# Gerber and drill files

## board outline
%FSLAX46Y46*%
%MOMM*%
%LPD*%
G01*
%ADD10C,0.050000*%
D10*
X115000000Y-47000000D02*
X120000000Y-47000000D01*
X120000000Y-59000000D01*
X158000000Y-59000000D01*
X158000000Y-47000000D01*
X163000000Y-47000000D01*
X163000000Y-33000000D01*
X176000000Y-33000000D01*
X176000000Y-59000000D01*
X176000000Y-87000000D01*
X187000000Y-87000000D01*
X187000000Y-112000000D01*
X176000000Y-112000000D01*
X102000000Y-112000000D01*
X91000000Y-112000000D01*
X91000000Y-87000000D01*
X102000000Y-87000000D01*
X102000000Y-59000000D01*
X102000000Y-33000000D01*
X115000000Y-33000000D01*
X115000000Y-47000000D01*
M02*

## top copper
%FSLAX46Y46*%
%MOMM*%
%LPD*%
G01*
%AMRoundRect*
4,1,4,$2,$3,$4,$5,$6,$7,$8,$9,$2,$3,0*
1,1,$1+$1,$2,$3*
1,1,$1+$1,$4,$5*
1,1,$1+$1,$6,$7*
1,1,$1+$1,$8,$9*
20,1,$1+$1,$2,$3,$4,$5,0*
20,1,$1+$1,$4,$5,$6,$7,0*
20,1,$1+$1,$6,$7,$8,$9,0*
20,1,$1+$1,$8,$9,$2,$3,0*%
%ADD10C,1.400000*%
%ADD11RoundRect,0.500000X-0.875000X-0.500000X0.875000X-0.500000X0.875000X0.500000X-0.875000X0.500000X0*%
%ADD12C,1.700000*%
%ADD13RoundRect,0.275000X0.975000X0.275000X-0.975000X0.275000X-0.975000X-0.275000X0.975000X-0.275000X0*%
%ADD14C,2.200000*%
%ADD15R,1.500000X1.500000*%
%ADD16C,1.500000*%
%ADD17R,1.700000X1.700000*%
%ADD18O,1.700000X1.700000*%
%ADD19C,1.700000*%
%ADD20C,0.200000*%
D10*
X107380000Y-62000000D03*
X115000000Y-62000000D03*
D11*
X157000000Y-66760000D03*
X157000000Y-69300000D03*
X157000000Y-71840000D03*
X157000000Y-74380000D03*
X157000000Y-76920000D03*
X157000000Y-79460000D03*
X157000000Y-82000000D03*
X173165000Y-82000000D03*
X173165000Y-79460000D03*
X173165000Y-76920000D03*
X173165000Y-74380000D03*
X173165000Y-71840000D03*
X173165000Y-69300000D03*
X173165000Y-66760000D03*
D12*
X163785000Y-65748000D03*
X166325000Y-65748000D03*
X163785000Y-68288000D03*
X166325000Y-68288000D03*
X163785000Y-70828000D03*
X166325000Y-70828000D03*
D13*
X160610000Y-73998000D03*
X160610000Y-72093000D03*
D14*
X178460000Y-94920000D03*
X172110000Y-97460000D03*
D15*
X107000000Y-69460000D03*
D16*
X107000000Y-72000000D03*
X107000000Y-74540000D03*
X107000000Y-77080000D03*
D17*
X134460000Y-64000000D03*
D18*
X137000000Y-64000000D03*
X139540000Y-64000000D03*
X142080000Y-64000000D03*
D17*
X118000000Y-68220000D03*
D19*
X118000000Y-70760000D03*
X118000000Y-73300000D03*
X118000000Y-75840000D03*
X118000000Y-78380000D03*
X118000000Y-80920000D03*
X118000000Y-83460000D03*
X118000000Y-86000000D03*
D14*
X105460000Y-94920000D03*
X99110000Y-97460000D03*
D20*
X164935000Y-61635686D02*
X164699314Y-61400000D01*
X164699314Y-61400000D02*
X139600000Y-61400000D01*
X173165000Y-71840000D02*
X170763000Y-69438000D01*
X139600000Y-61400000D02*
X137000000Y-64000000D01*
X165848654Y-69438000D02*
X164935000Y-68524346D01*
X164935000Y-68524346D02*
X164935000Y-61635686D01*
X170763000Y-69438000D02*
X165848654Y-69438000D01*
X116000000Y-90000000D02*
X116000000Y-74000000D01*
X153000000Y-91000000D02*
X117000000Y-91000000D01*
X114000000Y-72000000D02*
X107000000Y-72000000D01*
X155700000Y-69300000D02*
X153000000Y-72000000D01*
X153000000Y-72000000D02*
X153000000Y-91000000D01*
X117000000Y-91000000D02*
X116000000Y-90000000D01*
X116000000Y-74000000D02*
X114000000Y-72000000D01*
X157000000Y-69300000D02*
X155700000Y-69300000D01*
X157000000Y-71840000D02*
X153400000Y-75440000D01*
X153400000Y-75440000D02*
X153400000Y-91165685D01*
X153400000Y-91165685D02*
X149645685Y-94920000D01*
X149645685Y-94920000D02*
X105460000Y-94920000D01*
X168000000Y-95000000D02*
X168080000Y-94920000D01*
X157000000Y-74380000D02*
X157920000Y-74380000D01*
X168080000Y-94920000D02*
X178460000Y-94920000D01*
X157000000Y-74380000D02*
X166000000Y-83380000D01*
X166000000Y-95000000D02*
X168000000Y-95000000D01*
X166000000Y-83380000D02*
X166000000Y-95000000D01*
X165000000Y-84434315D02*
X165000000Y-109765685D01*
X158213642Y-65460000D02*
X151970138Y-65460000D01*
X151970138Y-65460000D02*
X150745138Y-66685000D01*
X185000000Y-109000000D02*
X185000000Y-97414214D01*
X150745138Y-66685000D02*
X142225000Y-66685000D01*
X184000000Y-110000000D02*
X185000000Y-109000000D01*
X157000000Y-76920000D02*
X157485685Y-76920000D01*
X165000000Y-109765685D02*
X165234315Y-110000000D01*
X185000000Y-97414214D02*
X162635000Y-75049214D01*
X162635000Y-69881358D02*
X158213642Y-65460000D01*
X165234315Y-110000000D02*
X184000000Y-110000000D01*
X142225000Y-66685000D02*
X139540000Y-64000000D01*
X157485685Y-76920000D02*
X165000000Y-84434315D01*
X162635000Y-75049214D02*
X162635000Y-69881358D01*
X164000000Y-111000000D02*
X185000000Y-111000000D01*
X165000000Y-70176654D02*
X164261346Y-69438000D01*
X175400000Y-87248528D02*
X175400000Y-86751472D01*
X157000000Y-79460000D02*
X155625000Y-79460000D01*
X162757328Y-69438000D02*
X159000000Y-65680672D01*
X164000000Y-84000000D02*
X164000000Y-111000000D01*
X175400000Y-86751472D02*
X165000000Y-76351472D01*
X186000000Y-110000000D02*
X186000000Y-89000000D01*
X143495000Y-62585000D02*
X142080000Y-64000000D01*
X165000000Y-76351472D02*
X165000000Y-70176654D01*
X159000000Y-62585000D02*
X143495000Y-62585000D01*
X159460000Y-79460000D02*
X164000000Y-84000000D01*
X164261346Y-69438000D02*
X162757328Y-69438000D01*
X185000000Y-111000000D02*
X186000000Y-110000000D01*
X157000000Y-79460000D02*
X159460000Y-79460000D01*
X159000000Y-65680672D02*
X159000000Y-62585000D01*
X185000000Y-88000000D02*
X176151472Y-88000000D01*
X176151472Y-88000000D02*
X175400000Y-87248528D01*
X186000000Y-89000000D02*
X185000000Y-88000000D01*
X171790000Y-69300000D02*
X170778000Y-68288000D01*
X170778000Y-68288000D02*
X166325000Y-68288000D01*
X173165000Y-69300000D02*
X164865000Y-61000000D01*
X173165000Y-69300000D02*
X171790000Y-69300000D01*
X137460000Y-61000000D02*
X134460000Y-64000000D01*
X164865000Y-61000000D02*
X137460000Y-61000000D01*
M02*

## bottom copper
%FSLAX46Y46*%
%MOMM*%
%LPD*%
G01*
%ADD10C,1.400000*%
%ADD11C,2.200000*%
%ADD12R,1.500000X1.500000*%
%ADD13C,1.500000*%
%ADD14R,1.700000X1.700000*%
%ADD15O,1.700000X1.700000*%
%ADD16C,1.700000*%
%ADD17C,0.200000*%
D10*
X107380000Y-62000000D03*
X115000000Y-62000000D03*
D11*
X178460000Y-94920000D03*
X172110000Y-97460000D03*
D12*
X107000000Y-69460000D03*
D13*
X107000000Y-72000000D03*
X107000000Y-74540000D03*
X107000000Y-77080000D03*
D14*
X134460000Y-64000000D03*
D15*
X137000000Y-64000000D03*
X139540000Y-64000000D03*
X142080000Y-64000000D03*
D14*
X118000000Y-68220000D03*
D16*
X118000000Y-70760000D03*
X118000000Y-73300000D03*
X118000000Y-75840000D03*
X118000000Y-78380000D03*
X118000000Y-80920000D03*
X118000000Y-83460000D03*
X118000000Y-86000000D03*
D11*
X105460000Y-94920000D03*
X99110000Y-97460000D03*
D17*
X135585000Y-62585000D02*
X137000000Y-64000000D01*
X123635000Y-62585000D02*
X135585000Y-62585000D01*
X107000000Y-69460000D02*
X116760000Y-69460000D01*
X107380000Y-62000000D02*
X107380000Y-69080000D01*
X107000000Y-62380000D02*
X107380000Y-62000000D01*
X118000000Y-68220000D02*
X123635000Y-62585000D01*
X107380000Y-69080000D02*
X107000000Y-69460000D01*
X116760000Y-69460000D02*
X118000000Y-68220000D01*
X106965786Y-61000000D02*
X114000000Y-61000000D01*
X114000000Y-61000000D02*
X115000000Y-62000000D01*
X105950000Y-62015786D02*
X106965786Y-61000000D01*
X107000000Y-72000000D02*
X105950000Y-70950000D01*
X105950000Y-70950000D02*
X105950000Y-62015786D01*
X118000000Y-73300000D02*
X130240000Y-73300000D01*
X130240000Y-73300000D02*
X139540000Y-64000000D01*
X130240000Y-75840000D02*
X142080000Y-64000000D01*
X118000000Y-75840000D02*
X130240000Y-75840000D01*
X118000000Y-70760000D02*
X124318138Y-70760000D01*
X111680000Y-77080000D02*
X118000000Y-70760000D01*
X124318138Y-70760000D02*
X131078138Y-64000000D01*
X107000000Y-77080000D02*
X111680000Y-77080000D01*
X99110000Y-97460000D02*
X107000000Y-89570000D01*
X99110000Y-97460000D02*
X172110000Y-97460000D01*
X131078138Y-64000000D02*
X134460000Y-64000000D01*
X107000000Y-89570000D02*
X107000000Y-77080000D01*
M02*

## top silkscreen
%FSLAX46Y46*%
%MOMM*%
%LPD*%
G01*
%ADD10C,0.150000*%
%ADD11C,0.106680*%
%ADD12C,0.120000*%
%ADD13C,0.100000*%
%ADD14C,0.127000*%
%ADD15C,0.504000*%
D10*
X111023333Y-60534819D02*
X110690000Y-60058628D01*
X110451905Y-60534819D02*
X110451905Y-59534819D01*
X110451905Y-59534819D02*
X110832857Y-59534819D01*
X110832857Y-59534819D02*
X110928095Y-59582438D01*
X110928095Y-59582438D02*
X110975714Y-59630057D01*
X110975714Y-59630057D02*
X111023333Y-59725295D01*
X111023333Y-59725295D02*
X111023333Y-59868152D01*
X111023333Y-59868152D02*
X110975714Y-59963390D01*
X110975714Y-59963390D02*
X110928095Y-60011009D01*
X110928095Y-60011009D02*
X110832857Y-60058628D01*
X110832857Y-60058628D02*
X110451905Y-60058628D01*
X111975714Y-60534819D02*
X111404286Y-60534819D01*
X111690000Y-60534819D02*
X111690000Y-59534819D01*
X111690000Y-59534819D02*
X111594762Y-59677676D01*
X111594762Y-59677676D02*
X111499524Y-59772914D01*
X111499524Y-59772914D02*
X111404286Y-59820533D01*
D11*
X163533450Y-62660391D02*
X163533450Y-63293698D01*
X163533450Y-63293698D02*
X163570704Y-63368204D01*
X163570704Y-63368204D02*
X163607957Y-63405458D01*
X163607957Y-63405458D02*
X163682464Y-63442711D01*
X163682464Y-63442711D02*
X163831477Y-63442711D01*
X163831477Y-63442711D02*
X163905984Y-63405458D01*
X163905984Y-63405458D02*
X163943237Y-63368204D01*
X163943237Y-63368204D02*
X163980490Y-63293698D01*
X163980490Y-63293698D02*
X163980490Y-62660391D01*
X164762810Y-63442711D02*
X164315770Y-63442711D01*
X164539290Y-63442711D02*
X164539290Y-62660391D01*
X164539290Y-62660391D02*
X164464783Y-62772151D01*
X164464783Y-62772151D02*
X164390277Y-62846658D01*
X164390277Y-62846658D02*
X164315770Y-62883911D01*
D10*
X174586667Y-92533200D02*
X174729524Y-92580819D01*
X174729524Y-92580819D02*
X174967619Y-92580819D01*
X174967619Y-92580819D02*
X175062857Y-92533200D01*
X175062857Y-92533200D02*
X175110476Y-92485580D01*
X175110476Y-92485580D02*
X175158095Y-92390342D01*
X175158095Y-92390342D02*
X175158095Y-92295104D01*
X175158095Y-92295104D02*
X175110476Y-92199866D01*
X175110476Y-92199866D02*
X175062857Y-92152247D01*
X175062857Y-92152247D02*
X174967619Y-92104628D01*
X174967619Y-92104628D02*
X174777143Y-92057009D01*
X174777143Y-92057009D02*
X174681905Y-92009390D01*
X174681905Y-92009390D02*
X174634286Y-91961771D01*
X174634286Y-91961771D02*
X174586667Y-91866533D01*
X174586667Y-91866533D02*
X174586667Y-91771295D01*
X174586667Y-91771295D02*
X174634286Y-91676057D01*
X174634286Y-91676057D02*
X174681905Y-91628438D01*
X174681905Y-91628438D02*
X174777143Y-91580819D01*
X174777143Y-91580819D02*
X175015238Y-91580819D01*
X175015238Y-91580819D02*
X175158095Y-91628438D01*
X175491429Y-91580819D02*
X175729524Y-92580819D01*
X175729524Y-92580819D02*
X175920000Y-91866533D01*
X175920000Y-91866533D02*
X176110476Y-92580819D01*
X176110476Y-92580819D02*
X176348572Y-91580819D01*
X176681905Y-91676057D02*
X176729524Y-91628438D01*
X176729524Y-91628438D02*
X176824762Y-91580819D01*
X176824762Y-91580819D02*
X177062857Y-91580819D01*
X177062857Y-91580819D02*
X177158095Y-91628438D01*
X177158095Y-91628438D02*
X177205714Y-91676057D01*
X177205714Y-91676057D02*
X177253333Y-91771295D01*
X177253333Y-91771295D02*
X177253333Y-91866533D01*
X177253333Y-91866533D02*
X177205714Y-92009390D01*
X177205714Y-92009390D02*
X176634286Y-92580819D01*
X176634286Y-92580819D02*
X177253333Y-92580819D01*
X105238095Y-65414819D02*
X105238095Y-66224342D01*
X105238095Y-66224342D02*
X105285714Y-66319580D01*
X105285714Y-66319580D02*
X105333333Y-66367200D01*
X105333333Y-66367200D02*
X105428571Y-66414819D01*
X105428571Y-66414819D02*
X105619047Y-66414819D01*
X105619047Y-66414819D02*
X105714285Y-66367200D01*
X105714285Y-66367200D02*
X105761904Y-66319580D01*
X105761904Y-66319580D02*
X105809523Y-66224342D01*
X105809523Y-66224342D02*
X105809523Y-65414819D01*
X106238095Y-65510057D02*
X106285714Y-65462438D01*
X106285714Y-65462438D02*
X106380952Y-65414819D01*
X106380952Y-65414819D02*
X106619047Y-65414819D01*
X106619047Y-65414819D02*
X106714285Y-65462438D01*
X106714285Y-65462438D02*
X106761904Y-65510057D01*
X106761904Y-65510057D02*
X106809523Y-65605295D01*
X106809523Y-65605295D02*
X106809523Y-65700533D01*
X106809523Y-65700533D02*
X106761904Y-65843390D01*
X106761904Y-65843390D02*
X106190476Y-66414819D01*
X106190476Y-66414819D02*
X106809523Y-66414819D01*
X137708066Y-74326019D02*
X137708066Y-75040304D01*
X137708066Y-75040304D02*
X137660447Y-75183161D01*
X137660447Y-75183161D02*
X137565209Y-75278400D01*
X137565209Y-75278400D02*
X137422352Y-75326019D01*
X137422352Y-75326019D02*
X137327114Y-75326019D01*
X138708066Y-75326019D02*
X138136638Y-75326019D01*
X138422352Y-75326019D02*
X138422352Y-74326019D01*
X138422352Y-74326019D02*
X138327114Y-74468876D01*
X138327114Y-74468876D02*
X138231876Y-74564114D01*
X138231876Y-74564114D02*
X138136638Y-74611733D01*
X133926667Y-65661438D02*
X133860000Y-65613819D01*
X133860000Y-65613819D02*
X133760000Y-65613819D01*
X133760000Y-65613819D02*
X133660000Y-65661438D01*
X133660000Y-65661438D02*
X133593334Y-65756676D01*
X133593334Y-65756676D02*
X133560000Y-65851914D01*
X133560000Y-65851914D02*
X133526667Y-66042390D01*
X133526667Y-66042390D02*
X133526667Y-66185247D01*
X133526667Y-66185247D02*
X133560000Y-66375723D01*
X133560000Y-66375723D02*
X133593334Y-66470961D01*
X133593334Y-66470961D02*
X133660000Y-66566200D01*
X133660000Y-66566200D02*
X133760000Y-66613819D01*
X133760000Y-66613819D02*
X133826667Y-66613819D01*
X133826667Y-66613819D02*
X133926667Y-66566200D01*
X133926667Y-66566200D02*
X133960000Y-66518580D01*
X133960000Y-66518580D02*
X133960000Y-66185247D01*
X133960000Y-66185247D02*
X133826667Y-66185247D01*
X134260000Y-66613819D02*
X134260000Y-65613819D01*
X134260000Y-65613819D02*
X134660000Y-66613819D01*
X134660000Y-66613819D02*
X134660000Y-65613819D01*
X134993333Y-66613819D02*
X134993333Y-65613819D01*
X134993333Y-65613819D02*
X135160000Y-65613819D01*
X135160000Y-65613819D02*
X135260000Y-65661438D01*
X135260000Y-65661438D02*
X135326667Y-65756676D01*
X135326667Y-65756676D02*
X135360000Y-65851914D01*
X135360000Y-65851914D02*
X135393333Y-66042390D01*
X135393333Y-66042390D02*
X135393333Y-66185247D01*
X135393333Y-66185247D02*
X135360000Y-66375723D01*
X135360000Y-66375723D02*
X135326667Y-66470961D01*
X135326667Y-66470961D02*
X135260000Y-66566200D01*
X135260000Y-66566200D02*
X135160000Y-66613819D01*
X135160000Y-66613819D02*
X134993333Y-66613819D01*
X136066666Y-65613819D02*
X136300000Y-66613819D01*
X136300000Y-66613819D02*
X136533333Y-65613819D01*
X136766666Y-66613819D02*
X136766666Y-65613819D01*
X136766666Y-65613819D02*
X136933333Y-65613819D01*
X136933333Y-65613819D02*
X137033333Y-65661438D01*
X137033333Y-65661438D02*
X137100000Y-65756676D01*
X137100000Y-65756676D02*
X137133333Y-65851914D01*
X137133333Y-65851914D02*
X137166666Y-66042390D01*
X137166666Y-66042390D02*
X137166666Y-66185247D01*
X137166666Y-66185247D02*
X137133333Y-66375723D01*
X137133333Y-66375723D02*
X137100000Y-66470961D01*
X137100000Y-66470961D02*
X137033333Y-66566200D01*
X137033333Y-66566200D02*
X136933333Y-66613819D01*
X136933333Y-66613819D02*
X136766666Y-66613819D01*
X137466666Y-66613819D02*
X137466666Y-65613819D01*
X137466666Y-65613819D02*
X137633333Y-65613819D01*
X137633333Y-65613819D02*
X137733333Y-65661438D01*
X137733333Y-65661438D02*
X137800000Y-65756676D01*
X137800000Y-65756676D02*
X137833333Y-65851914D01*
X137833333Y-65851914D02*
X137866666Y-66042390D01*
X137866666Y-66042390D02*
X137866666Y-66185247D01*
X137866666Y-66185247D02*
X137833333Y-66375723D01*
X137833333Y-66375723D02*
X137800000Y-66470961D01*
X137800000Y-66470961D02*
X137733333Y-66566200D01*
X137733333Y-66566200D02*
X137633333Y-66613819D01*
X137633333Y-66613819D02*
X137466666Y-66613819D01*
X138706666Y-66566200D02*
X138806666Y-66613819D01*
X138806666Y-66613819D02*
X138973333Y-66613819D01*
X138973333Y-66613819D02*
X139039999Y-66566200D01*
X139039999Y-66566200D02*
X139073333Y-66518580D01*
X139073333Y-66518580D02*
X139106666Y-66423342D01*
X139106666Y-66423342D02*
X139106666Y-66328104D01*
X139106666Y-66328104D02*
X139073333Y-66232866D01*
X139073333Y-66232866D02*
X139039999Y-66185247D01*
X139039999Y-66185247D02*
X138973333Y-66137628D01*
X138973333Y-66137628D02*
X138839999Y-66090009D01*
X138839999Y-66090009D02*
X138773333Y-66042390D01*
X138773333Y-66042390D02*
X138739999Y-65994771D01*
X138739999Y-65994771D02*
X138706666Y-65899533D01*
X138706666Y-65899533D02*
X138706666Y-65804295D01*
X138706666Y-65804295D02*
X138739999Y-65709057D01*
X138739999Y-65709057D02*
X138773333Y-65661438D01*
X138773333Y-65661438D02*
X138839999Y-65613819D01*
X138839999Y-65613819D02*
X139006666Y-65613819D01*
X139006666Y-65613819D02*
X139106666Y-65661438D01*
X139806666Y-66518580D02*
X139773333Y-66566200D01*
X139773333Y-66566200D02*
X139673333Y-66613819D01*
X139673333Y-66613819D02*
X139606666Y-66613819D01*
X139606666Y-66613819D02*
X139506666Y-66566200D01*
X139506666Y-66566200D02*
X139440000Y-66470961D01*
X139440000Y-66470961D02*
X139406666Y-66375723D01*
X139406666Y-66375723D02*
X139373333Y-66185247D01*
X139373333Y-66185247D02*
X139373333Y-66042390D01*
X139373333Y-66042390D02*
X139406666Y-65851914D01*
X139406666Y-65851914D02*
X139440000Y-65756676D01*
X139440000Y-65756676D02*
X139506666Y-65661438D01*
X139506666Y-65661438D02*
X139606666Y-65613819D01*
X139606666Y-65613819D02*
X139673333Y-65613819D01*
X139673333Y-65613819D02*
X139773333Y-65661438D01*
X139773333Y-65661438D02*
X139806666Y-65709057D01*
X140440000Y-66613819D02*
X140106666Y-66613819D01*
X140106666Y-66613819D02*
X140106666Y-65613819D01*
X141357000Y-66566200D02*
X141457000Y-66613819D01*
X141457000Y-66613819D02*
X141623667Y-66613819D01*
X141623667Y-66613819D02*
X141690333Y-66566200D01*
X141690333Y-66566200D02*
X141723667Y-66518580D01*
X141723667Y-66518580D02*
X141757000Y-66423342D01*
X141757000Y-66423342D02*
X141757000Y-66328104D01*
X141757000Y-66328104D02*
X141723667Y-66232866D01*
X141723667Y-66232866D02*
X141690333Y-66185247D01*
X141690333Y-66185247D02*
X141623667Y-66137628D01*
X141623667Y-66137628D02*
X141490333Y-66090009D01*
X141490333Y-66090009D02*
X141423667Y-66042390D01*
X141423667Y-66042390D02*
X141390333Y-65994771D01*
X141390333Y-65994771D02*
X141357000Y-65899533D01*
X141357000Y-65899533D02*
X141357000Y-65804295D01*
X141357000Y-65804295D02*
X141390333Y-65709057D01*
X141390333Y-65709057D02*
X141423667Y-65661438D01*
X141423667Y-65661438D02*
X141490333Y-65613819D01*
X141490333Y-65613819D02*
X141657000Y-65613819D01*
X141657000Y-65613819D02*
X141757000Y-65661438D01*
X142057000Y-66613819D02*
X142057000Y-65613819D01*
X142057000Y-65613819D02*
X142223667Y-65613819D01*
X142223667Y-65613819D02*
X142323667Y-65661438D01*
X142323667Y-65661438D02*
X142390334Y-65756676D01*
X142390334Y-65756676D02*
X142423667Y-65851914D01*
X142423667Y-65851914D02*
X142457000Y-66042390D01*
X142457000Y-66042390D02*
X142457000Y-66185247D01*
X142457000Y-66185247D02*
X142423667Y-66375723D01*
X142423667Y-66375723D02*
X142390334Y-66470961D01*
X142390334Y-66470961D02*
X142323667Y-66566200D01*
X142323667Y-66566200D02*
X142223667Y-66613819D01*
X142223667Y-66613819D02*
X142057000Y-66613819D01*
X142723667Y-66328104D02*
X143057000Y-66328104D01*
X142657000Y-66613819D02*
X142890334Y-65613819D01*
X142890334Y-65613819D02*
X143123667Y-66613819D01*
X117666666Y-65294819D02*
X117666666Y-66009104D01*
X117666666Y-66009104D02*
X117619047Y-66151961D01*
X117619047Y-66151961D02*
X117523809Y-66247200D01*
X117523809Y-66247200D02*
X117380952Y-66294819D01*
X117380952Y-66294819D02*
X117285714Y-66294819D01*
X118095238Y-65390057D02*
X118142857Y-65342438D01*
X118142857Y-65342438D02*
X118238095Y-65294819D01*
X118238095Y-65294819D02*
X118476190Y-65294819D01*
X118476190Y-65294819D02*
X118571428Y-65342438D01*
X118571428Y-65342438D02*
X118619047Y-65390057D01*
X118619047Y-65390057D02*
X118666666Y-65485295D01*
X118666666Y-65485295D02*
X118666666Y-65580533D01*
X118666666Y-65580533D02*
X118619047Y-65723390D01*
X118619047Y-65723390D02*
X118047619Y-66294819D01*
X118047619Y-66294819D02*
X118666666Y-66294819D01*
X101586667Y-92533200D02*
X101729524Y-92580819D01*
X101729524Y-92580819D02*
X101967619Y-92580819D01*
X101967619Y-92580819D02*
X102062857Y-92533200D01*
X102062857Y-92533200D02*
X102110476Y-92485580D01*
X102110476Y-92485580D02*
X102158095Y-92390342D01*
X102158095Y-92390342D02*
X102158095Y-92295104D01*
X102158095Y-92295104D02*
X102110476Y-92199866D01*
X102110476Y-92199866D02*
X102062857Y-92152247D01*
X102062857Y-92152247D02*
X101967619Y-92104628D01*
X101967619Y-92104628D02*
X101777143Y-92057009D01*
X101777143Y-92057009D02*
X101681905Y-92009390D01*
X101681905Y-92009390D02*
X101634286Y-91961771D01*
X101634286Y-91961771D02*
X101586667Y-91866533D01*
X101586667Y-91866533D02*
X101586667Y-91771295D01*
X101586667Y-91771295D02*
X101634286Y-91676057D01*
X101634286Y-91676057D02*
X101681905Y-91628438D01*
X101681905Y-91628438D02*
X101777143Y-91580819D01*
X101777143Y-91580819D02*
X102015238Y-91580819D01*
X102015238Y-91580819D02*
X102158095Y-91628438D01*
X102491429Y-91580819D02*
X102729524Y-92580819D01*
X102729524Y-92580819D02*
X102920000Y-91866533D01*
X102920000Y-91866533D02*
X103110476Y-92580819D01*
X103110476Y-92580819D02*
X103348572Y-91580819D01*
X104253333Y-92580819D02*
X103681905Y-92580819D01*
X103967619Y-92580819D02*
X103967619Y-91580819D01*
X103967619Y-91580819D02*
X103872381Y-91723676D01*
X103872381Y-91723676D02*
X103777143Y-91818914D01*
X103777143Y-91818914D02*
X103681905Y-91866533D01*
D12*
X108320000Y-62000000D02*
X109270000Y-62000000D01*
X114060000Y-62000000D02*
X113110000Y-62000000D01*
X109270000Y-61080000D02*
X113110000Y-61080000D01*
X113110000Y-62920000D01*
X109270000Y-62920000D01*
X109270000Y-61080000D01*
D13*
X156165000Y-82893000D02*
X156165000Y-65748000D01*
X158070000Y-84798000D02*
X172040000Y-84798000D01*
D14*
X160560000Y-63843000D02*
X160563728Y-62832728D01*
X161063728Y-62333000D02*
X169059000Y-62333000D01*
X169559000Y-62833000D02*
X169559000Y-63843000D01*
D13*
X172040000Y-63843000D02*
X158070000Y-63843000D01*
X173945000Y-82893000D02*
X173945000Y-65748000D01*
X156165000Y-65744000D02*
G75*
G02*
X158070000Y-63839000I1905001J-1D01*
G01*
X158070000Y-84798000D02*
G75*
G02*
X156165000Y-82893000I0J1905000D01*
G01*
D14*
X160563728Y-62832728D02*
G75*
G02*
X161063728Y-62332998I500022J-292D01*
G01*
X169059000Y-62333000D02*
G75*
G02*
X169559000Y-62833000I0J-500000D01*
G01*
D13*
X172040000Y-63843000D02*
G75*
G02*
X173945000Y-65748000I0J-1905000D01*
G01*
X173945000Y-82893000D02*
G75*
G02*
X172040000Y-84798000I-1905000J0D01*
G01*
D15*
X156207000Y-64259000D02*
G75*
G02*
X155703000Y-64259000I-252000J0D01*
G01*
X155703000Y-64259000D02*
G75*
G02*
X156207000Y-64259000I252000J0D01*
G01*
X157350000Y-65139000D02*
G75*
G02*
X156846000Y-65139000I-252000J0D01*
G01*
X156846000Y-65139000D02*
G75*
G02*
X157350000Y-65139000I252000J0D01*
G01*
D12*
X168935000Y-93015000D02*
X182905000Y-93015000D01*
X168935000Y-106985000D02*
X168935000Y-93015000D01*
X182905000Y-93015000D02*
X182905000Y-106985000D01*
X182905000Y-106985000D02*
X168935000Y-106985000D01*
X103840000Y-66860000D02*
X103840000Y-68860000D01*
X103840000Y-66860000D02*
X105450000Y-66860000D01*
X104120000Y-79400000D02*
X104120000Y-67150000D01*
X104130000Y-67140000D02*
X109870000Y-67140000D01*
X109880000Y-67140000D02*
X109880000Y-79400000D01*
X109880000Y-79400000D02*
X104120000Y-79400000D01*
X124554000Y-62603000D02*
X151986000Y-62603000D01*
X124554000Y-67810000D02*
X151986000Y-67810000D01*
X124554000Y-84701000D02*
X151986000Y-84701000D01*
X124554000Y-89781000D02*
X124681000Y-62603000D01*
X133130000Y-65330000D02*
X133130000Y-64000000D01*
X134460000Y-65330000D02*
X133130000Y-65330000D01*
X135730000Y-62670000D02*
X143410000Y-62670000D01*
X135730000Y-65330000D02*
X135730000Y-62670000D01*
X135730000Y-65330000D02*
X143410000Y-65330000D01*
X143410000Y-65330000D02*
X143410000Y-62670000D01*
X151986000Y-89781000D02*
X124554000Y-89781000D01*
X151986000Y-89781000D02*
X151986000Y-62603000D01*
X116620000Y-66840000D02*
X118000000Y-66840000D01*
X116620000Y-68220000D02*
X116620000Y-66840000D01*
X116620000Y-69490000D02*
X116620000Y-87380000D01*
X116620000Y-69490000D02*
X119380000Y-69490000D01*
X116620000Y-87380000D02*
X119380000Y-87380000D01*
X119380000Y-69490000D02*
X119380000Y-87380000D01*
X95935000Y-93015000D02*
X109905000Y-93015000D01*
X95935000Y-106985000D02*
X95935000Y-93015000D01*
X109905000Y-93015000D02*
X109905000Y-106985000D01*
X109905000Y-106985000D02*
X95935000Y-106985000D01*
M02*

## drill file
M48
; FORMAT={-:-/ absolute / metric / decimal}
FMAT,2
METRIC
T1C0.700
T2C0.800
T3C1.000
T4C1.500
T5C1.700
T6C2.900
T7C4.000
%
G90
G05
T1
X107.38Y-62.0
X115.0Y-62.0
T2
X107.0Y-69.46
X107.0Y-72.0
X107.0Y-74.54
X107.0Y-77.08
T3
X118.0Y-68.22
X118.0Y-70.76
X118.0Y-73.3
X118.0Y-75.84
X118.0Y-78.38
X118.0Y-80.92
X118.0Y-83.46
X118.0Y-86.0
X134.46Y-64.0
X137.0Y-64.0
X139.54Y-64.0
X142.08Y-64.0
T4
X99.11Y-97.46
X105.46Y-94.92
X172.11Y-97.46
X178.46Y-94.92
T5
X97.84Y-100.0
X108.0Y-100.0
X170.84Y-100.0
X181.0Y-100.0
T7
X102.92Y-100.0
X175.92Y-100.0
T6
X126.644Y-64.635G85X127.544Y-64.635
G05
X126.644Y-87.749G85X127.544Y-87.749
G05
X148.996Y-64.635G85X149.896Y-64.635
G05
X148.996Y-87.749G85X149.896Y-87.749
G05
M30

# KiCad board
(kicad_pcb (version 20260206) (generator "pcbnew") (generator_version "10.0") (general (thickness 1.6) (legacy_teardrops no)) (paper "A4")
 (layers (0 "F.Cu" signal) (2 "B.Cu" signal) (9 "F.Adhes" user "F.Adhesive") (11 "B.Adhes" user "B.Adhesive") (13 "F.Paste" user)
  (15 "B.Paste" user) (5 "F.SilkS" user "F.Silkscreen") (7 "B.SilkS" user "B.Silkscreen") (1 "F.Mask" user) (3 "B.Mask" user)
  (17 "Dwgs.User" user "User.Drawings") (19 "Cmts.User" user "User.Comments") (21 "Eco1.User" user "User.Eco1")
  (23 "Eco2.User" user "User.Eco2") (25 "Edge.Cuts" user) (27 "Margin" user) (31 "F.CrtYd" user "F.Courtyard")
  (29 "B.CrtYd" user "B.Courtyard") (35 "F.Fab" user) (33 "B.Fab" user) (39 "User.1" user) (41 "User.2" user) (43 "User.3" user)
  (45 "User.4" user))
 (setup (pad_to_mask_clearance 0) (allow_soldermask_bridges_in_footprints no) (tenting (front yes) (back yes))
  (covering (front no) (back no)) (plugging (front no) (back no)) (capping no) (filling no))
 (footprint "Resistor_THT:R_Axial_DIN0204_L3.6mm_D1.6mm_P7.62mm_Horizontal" (layer "F.Cu") (at 107.38 62)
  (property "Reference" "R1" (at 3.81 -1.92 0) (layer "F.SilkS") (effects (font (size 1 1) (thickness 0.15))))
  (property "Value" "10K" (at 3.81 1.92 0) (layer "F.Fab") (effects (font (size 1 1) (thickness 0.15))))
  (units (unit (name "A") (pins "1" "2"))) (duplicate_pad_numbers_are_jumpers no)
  (fp_line (start 0.94 0) (end 1.89 0) (stroke (width 0.12) (type solid)) (layer "F.SilkS"))
  (fp_line (start 6.68 0) (end 5.73 0) (stroke (width 0.12) (type solid)) (layer "F.SilkS"))
  (fp_rect (start 1.89 -0.92) (end 5.73 0.92) (stroke (width 0.12) (type solid)) (fill no) (layer "F.SilkS"))
  (pad "1" thru_hole circle (at 0 0) (size 1.4 1.4) (drill 0.7) (layers "*.Cu" "*.Mask") (remove_unused_layers no) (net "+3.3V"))
  (pad "2" thru_hole circle (at 7.62 0) (size 1.4 1.4) (drill 0.7) (layers "*.Cu" "*.Mask") (remove_unused_layers no) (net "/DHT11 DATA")))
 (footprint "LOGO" (layer "F.Cu") (at 157 97)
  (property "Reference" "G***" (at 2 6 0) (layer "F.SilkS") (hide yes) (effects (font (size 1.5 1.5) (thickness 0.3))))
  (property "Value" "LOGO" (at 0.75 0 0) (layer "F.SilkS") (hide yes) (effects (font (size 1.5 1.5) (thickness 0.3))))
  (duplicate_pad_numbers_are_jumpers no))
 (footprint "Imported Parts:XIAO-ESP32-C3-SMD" (layer "F.Cu") (at 156.165 84.88)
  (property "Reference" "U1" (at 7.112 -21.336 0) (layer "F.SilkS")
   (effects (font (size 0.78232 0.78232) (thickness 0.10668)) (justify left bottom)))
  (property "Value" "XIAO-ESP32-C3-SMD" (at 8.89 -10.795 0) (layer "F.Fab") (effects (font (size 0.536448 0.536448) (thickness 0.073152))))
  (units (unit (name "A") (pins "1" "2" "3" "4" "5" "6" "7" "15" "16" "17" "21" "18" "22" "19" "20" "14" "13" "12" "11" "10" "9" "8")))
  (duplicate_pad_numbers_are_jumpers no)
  (fp_line (start 0 -1.987) (end 0 -19.132) (stroke (width 0.1) (type solid)) (layer "F.SilkS"))
  (fp_line (start 1.905 -0.082) (end 15.875 -0.082) (stroke (width 0.1) (type solid)) (layer "F.SilkS"))
  (fp_line (start 4.395 -21.037) (end 4.398728 -22.047272) (stroke (width 0.127) (type solid)) (layer "F.SilkS"))
  (fp_line (start 4.898728 -22.547) (end 12.894 -22.547) (stroke (width 0.127) (type solid)) (layer "F.SilkS"))
  (fp_line (start 13.394 -22.047) (end 13.394 -21.037) (stroke (width 0.127) (type solid)) (layer "F.SilkS"))
  (fp_line (start 15.875 -21.037) (end 1.905 -21.037) (stroke (width 0.1) (type solid)) (layer "F.SilkS"))
  (fp_line (start 17.78 -1.987) (end 17.78 -19.132) (stroke (width 0.1) (type solid)) (layer "F.SilkS"))
  (fp_arc (start 0 -19.136) (mid 0.557962 -20.483038) (end 1.905 -21.041) (stroke (width 0.1) (type solid)) (layer "F.SilkS"))
  (fp_arc (start 1.905 -0.082) (mid 0.557962 -0.639962) (end 0 -1.987) (stroke (width 0.1) (type solid)) (layer "F.SilkS"))
  (fp_arc (start 4.398728 -22.047272) (mid 4.545272 -22.40064) (end 4.898728 -22.547) (stroke (width 0.127) (type default))
   (layer "F.SilkS"))
  (fp_arc (start 12.894 -22.547) (mid 13.247553 -22.400553) (end 13.394 -22.047) (stroke (width 0.127) (type default)) (layer "F.SilkS"))
  (fp_arc (start 15.875 -21.037) (mid 17.222038 -20.479038) (end 17.78 -19.132) (stroke (width 0.1) (type solid)) (layer "F.SilkS"))
  (fp_arc (start 17.78 -1.987) (mid 17.222038 -0.639962) (end 15.875 -0.082) (stroke (width 0.1) (type solid)) (layer "F.SilkS"))
  (fp_circle (center -0.21 -20.621) (end -0.21 -20.875) (stroke (width 0.5) (type solid)) (fill yes) (layer "F.SilkS"))
  (fp_circle (center 0.933 -19.741) (end 0.933 -19.995) (stroke (width 0.5) (type solid)) (fill yes) (layer "F.SilkS"))
  (pad "1" smd roundrect (at 0.835 -18.12) (size 2.75 2) (layers "F.Cu" "F.Mask" "F.Paste") (roundrect_rratio 0.25)
   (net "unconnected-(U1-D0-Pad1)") (solder_mask_margin 0.0508) (thermal_bridge_angle 45))
  (pad "2" smd roundrect (at 0.835 -15.58) (size 2.75 2) (layers "F.Cu" "F.Mask" "F.Paste") (roundrect_rratio 0.25) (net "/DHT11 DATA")
   (solder_mask_margin 0.0508) (thermal_bridge_angle 45))
  (pad "3" smd roundrect (at 0.835 -13.04) (size 2.75 2) (layers "F.Cu" "F.Mask" "F.Paste") (roundrect_rratio 0.25) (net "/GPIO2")
   (solder_mask_margin 0.0508) (thermal_bridge_angle 45))
  (pad "4" smd roundrect (at 0.835 -10.5) (size 2.75 2) (layers "F.Cu" "F.Mask" "F.Paste") (roundrect_rratio 0.25) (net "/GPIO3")
   (solder_mask_margin 0.0508) (thermal_bridge_angle 45))
  (pad "5" smd roundrect (at 0.835 -7.96) (size 2.75 2) (layers "F.Cu" "F.Mask" "F.Paste") (roundrect_rratio 0.25) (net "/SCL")
   (solder_mask_margin 0.0508) (thermal_bridge_angle 45))
  (pad "6" smd roundrect (at 0.835 -5.42) (size 2.75 2) (layers "F.Cu" "F.Mask" "F.Paste") (roundrect_rratio 0.25) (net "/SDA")
   (solder_mask_margin 0.0508) (thermal_bridge_angle 45))
  (pad "7" smd roundrect (at 0.835 -2.88) (size 2.75 2) (layers "F.Cu" "F.Mask" "F.Paste") (roundrect_rratio 0.25)
   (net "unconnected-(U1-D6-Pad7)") (solder_mask_margin 0.0508) (thermal_bridge_angle 45))
  (pad "8" smd roundrect (at 17 -2.88) (size 2.75 2) (layers "F.Cu" "F.Mask" "F.Paste") (roundrect_rratio 0.25)
   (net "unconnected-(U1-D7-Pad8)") (solder_mask_margin 0.0508) (thermal_bridge_angle 45))
  (pad "9" smd roundrect (at 17 -5.42) (size 2.75 2) (layers "F.Cu" "F.Mask" "F.Paste") (roundrect_rratio 0.25)
   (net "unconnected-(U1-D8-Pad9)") (solder_mask_margin 0.0508) (thermal_bridge_angle 45))
  (pad "10" smd roundrect (at 17 -7.96) (size 2.75 2) (layers "F.Cu" "F.Mask" "F.Paste") (roundrect_rratio 0.25)
   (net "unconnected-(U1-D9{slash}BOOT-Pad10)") (solder_mask_margin 0.0508) (thermal_bridge_angle 45))
  (pad "11" smd roundrect (at 17 -10.5) (size 2.75 2) (layers "F.Cu" "F.Mask" "F.Paste") (roundrect_rratio 0.25)
   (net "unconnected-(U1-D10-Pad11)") (solder_mask_margin 0.0508) (thermal_bridge_angle 45))
  (pad "12" smd roundrect (at 17 -13.04) (size 2.75 2) (layers "F.Cu" "F.Mask" "F.Paste") (roundrect_rratio 0.25) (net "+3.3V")
   (solder_mask_margin 0.0508) (thermal_bridge_angle 45))
  (pad "13" smd roundrect (at 17 -15.58) (size 2.75 2) (layers "F.Cu" "F.Mask" "F.Paste") (roundrect_rratio 0.25) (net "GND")
   (solder_mask_margin 0.0508) (thermal_bridge_angle 45))
  (pad "14" smd roundrect (at 17 -18.12) (size 2.75 2) (layers "F.Cu" "F.Mask" "F.Paste") (roundrect_rratio 0.25) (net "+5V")
   (solder_mask_margin 0.0508) (thermal_bridge_angle 45))
  (pad "15" smd circle (at 7.62 -19.132) (size 1.7 1.7) (layers "F.Cu" "F.Mask" "F.Paste") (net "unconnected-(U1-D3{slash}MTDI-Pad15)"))
  (pad "16" smd circle (at 10.16 -19.132) (size 1.7 1.7) (layers "F.Cu" "F.Mask" "F.Paste") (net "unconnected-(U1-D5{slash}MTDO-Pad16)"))
  (pad "17" smd circle (at 7.62 -16.592) (size 1.7 1.7) (layers "F.Cu" "F.Mask" "F.Paste") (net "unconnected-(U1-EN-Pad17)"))
  (pad "18" smd circle (at 10.16 -16.592) (size 1.7 1.7) (layers "F.Cu" "F.Mask" "F.Paste") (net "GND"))
  (pad "19" smd circle (at 7.62 -14.052) (size 1.7 1.7) (layers "F.Cu" "F.Mask" "F.Paste") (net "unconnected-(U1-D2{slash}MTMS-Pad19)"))
  (pad "20" smd circle (at 10.16 -14.052) (size 1.7 1.7) (layers "F.Cu" "F.Mask" "F.Paste") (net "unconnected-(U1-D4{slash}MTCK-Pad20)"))
  (pad "21" smd roundrect (at 4.445 -10.882 180) (size 2.5 1.1) (layers "F.Cu" "F.Mask" "F.Paste") (roundrect_rratio 0.25)
   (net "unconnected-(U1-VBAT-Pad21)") (thermal_bridge_angle 45))
  (pad "22" smd roundrect (at 4.445 -12.787 180) (size 2.5 1.1) (layers "F.Cu" "F.Mask" "F.Paste") (roundrect_rratio 0.25)
   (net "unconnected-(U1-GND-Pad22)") (thermal_bridge_angle 45)))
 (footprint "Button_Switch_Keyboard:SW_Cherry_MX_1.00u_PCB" (layer "F.Cu") (at 178.46 94.92)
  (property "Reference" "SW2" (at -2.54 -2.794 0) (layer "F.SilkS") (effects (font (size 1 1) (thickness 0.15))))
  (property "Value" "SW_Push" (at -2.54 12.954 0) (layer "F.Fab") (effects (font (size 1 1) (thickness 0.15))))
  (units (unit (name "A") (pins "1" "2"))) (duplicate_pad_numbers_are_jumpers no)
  (fp_line (start -9.525 -1.905) (end 4.445 -1.905) (stroke (width 0.12) (type solid)) (layer "F.SilkS"))
  (fp_line (start -9.525 12.065) (end -9.525 -1.905) (stroke (width 0.12) (type solid)) (layer "F.SilkS"))
  (fp_line (start 4.445 -1.905) (end 4.445 12.065) (stroke (width 0.12) (type solid)) (layer "F.SilkS"))
  (fp_line (start 4.445 12.065) (end -9.525 12.065) (stroke (width 0.12) (type solid)) (layer "F.SilkS"))
  (pad "" np_thru_hole circle (at -7.62 5.08) (size 1.7 1.7) (drill 1.7) (layers "*.Cu" "*.Mask"))
  (pad "" np_thru_hole circle (at -2.54 5.08) (size 4 4) (drill 4) (layers "*.Cu" "*.Mask"))
  (pad "" np_thru_hole circle (at 2.54 5.08) (size 1.7 1.7) (drill 1.7) (layers "*.Cu" "*.Mask"))
  (pad "1" thru_hole circle (at 0 0) (size 2.2 2.2) (drill 1.5) (layers "*.Cu" "*.Mask") (remove_unused_layers no) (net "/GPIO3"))
  (pad "2" thru_hole circle (at -6.35 2.54) (size 2.2 2.2) (drill 1.5) (layers "*.Cu" "*.Mask") (remove_unused_layers no) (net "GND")))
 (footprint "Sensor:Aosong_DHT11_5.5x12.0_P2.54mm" (layer "F.Cu") (at 107 69.46)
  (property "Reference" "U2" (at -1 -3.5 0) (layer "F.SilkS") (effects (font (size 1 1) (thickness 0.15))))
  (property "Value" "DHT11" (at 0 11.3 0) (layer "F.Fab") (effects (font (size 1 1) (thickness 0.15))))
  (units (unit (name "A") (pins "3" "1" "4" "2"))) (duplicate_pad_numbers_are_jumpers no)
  (fp_line (start -3.16 -2.6) (end -3.16 -0.6) (stroke (width 0.12) (type solid)) (layer "F.SilkS"))
  (fp_line (start -3.16 -2.6) (end -1.55 -2.6) (stroke (width 0.12) (type solid)) (layer "F.SilkS"))
  (fp_line (start -2.88 9.94) (end -2.88 -2.31) (stroke (width 0.12) (type solid)) (layer "F.SilkS"))
  (fp_line (start -2.87 -2.32) (end 2.87 -2.32) (stroke (width 0.12) (type solid)) (layer "F.SilkS"))
  (fp_line (start 2.88 -2.32) (end 2.88 9.94) (stroke (width 0.12) (type solid)) (layer "F.SilkS"))
  (fp_line (start 2.88 9.94) (end -2.88 9.94) (stroke (width 0.12) (type solid)) (layer "F.SilkS"))
  (pad "1" thru_hole rect (at 0 0) (size 1.5 1.5) (drill 0.8) (layers "*.Cu" "*.Mask") (remove_unused_layers no) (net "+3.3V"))
  (pad "2" thru_hole circle (at 0 2.54) (size 1.5 1.5) (drill 0.8) (layers "*.Cu" "*.Mask") (remove_unused_layers no) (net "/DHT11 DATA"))
  (pad "3" thru_hole circle (at 0 5.08) (size 1.5 1.5) (drill 0.8) (layers "*.Cu" "*.Mask") (remove_unused_layers no)
   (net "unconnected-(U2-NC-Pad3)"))
  (pad "4" thru_hole circle (at 0 7.62) (size 1.5 1.5) (drill 0.8) (layers "*.Cu" "*.Mask") (remove_unused_layers no) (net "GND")))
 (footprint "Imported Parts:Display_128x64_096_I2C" (layer "F.Cu") (at 138.27 64)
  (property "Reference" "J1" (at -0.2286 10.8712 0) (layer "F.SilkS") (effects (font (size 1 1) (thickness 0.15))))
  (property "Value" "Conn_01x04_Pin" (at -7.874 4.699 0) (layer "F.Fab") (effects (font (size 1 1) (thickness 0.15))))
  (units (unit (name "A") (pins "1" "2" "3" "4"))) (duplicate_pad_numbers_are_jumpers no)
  (fp_line (start -13.716 -1.397) (end 13.716 -1.397) (stroke (width 0.12) (type solid)) (layer "F.SilkS"))
  (fp_line (start -13.716 3.81) (end 13.716 3.81) (stroke (width 0.12) (type solid)) (layer "F.SilkS"))
  (fp_line (start -13.716 20.701) (end 13.716 20.701) (stroke (width 0.12) (type solid)) (layer "F.SilkS"))
  (fp_line (start -13.716 25.781) (end -13.589 -1.397) (stroke (width 0.12) (type solid)) (layer "F.SilkS"))
  (fp_line (start -5.14 1.33) (end -5.14 0) (stroke (width 0.12) (type solid)) (layer "F.SilkS"))
  (fp_line (start -3.81 1.33) (end -5.14 1.33) (stroke (width 0.12) (type solid)) (layer "F.SilkS"))
  (fp_line (start -2.54 -1.33) (end 5.14 -1.33) (stroke (width 0.12) (type solid)) (layer "F.SilkS"))
  (fp_line (start -2.54 1.33) (end -2.54 -1.33) (stroke (width 0.12) (type solid)) (layer "F.SilkS"))
  (fp_line (start -2.54 1.33) (end 5.14 1.33) (stroke (width 0.12) (type solid)) (layer "F.SilkS"))
  (fp_line (start 5.14 1.33) (end 5.14 -1.33) (stroke (width 0.12) (type solid)) (layer "F.SilkS"))
  (fp_line (start 13.716 25.781) (end -13.716 25.781) (stroke (width 0.12) (type solid)) (layer "F.SilkS"))
  (fp_line (start 13.716 25.781) (end 13.716 -1.397) (stroke (width 0.12) (type solid)) (layer "F.SilkS"))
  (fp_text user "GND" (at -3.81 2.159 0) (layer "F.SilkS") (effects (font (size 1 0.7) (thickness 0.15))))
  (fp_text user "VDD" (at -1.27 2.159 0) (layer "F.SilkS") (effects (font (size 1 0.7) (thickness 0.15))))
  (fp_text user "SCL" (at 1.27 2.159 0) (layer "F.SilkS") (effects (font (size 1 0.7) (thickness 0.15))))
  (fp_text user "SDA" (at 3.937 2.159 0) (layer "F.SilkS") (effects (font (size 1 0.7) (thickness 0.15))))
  (pad "" np_thru_hole oval (at -11.176 0.635) (size 3.8 2.9) (drill oval 3.8 2.9) (layers "*.Cu" "*.Mask"))
  (pad "" np_thru_hole oval (at -11.176 23.749) (size 3.8 2.9) (drill oval 3.8 2.9) (layers "*.Cu" "*.Mask"))
  (pad "" np_thru_hole oval (at 11.176 0.635) (size 3.8 2.9) (drill oval 3.8 2.9) (layers "*.Cu" "*.Mask"))
  (pad "" np_thru_hole oval (at 11.176 23.749) (size 3.8 2.9) (drill oval 3.8 2.9) (layers "*.Cu" "*.Mask"))
  (pad "1" thru_hole rect (at -3.81 0 90) (size 1.7 1.7) (drill 1) (layers "*.Cu" "*.Mask") (remove_unused_layers no) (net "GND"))
  (pad "2" thru_hole oval (at -1.27 0 90) (size 1.7 1.7) (drill 1) (layers "*.Cu" "*.Mask") (remove_unused_layers no) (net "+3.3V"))
  (pad "3" thru_hole oval (at 1.27 0 90) (size 1.7 1.7) (drill 1) (layers "*.Cu" "*.Mask") (remove_unused_layers no) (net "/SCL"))
  (pad "4" thru_hole oval (at 3.81 0 90) (size 1.7 1.7) (drill 1) (layers "*.Cu" "*.Mask") (remove_unused_layers no) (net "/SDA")))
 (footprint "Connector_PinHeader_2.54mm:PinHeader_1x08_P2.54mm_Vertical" (layer "F.Cu") (at 118 68.22)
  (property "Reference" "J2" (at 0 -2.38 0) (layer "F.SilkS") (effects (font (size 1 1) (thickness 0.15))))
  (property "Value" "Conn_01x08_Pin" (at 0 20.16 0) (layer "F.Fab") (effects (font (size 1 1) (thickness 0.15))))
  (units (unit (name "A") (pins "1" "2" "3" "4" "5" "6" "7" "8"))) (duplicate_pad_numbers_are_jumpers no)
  (fp_line (start -1.38 -1.38) (end 0 -1.38) (stroke (width 0.12) (type solid)) (layer "F.SilkS"))
  (fp_line (start -1.38 0) (end -1.38 -1.38) (stroke (width 0.12) (type solid)) (layer "F.SilkS"))
  (fp_line (start -1.38 1.27) (end -1.38 19.16) (stroke (width 0.12) (type solid)) (layer "F.SilkS"))
  (fp_line (start -1.38 1.27) (end 1.38 1.27) (stroke (width 0.12) (type solid)) (layer "F.SilkS"))
  (fp_line (start -1.38 19.16) (end 1.38 19.16) (stroke (width 0.12) (type solid)) (layer "F.SilkS"))
  (fp_line (start 1.38 1.27) (end 1.38 19.16) (stroke (width 0.12) (type solid)) (layer "F.SilkS"))
  (pad "1" thru_hole rect (at 0 0) (size 1.7 1.7) (drill 1) (layers "*.Cu" "*.Mask") (remove_unused_layers no) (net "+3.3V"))
  (pad "2" thru_hole circle (at 0 2.54) (size 1.7 1.7) (drill 1) (layers "*.Cu" "*.Mask") (remove_unused_layers no) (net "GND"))
  (pad "3" thru_hole circle (at 0 5.08) (size 1.7 1.7) (drill 1) (layers "*.Cu" "*.Mask") (remove_unused_layers no) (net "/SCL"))
  (pad "4" thru_hole circle (at 0 7.62) (size 1.7 1.7) (drill 1) (layers "*.Cu" "*.Mask") (remove_unused_layers no) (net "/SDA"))
  (pad "5" thru_hole circle (at 0 10.16) (size 1.7 1.7) (drill 1) (layers "*.Cu" "*.Mask") (remove_unused_layers no)
   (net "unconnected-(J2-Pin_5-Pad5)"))
  (pad "6" thru_hole circle (at 0 12.7) (size 1.7 1.7) (drill 1) (layers "*.Cu" "*.Mask") (remove_unused_layers no)
   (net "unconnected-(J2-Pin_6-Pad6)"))
  (pad "7" thru_hole circle (at 0 15.24) (size 1.7 1.7) (drill 1) (layers "*.Cu" "*.Mask") (remove_unused_layers no)
   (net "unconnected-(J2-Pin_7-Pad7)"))
  (pad "8" thru_hole circle (at 0 17.78) (size 1.7 1.7) (drill 1) (layers "*.Cu" "*.Mask") (remove_unused_layers no)
   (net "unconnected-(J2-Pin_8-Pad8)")))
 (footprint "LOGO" (layer "F.Cu") (at 144 97)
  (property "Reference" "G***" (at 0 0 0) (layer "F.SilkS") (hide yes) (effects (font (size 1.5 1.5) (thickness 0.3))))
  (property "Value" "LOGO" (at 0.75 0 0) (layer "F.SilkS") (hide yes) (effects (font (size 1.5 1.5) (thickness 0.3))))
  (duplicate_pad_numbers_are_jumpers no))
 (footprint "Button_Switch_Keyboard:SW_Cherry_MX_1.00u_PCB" (layer "F.Cu") (at 105.46 94.92)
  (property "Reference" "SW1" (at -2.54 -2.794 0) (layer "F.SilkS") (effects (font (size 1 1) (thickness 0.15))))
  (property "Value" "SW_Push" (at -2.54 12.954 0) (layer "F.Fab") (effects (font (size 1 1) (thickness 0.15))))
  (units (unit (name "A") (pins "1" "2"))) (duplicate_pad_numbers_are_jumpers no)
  (fp_line (start -9.525 -1.905) (end 4.445 -1.905) (stroke (width 0.12) (type solid)) (layer "F.SilkS"))
  (fp_line (start -9.525 12.065) (end -9.525 -1.905) (stroke (width 0.12) (type solid)) (layer "F.SilkS"))
  (fp_line (start 4.445 -1.905) (end 4.445 12.065) (stroke (width 0.12) (type solid)) (layer "F.SilkS"))
  (fp_line (start 4.445 12.065) (end -9.525 12.065) (stroke (width 0.12) (type solid)) (layer "F.SilkS"))
  (pad "" np_thru_hole circle (at -7.62 5.08) (size 1.7 1.7) (drill 1.7) (layers "*.Cu" "*.Mask"))
  (pad "" np_thru_hole circle (at -2.54 5.08) (size 4 4) (drill 4) (layers "*.Cu" "*.Mask"))
  (pad "" np_thru_hole circle (at 2.54 5.08) (size 1.7 1.7) (drill 1.7) (layers "*.Cu" "*.Mask"))
  (pad "1" thru_hole circle (at 0 0) (size 2.2 2.2) (drill 1.5) (layers "*.Cu" "*.Mask") (remove_unused_layers no) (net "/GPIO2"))
  (pad "2" thru_hole circle (at -6.35 2.54) (size 2.2 2.2) (drill 1.5) (layers "*.Cu" "*.Mask") (remove_unused_layers no) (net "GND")))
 (gr_poly
  (pts (xy 115 47) (xy 120 47) (xy 120 59) (xy 158 59) (xy 158 47) (xy 163 47) (xy 163 33) (xy 176 33) (xy 176 59) (xy 176 87) (xy 187 87)
   (xy 187 112) (xy 176 112) (xy 102 112) (xy 91 112) (xy 91 87) (xy 102 87) (xy 102 59) (xy 102 33) (xy 115 33))
  (stroke (width 0.05) (type default)) (fill no) (layer "Edge.Cuts"))
 (segment (start 164.935 61.635686) (end 164.699314 61.4) (width 0.2) (layer "F.Cu") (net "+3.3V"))
 (segment (start 164.699314 61.4) (end 139.6 61.4) (width 0.2) (layer "F.Cu") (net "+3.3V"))
 (segment (start 173.165 71.84) (end 170.763 69.438) (width 0.2) (layer "F.Cu") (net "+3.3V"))
 (segment (start 139.6 61.4) (end 137 64) (width 0.2) (layer "F.Cu") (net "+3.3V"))
 (segment (start 165.848654 69.438) (end 164.935 68.524346) (width 0.2) (layer "F.Cu") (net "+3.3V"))
 (segment (start 164.935 68.524346) (end 164.935 61.635686) (width 0.2) (layer "F.Cu") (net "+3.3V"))
 (segment (start 170.763 69.438) (end 165.848654 69.438) (width 0.2) (layer "F.Cu") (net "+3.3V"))
 (segment (start 135.585 62.585) (end 137 64) (width 0.2) (layer "B.Cu") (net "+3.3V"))
 (segment (start 123.635 62.585) (end 135.585 62.585) (width 0.2) (layer "B.Cu") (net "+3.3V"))
 (segment (start 107 69.46) (end 116.76 69.46) (width 0.2) (layer "B.Cu") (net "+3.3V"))
 (segment (start 107.38 62) (end 107.38 69.08) (width 0.2) (layer "B.Cu") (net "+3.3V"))
 (segment (start 107 62.38) (end 107.38 62) (width 0.2) (layer "B.Cu") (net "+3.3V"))
 (segment (start 118 68.22) (end 123.635 62.585) (width 0.2) (layer "B.Cu") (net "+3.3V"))
 (segment (start 107.38 69.08) (end 107 69.46) (width 0.2) (layer "B.Cu") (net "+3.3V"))
 (segment (start 116.76 69.46) (end 118 68.22) (width 0.2) (layer "B.Cu") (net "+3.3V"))
 (segment (start 116 90) (end 116 74) (width 0.2) (layer "F.Cu") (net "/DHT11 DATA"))
 (segment (start 153 91) (end 117 91) (width 0.2) (layer "F.Cu") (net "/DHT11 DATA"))
 (segment (start 114 72) (end 107 72) (width 0.2) (layer "F.Cu") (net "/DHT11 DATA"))
 (segment (start 155.7 69.3) (end 153 72) (width 0.2) (layer "F.Cu") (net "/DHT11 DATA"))
 (segment (start 153 72) (end 153 91) (width 0.2) (layer "F.Cu") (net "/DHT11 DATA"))
 (segment (start 117 91) (end 116 90) (width 0.2) (layer "F.Cu") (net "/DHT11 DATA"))
 (segment (start 116 74) (end 114 72) (width 0.2) (layer "F.Cu") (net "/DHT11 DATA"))
 (segment (start 157 69.3) (end 155.7 69.3) (width 0.2) (layer "F.Cu") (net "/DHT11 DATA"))
 (segment (start 106.965786 61) (end 114 61) (width 0.2) (layer "B.Cu") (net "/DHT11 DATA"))
 (segment (start 114 61) (end 115 62) (width 0.2) (layer "B.Cu") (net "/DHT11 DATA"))
 (segment (start 105.95 62.015786) (end 106.965786 61) (width 0.2) (layer "B.Cu") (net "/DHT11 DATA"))
 (segment (start 107 72) (end 105.95 70.95) (width 0.2) (layer "B.Cu") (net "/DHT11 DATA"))
 (segment (start 105.95 70.95) (end 105.95 62.015786) (width 0.2) (layer "B.Cu") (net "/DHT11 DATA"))
 (segment (start 157 71.84) (end 153.4 75.44) (width 0.2) (layer "F.Cu") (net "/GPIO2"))
 (segment (start 153.4 75.44) (end 153.4 91.165685) (width 0.2) (layer "F.Cu") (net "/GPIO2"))
 (segment (start 153.4 91.165685) (end 149.645685 94.92) (width 0.2) (layer "F.Cu") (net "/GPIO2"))
 (segment (start 149.645685 94.92) (end 105.46 94.92) (width 0.2) (layer "F.Cu") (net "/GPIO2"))
 (segment (start 168 95) (end 168.08 94.92) (width 0.2) (layer "F.Cu") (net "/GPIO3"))
 (segment (start 157 74.38) (end 157.92 74.38) (width 0.2) (layer "F.Cu") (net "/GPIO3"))
 (segment (start 168.08 94.92) (end 178.46 94.92) (width 0.2) (layer "F.Cu") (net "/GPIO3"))
 (segment (start 157 74.38) (end 166 83.38) (width 0.2) (layer "F.Cu") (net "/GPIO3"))
 (segment (start 166 95) (end 168 95) (width 0.2) (layer "F.Cu") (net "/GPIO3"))
 (segment (start 166 83.38) (end 166 95) (width 0.2) (layer "F.Cu") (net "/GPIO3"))
 (segment (start 165 84.434315) (end 165 109.765685) (width 0.2) (layer "F.Cu") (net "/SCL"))
 (segment (start 158.213642 65.46) (end 151.970138 65.46) (width 0.2) (layer "F.Cu") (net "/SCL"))
 (segment (start 151.970138 65.46) (end 150.745138 66.685) (width 0.2) (layer "F.Cu") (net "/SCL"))
 (segment (start 185 109) (end 185 97.414214) (width 0.2) (layer "F.Cu") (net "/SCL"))
 (segment (start 150.745138 66.685) (end 142.225 66.685) (width 0.2) (layer "F.Cu") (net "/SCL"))
 (segment (start 184 110) (end 185 109) (width 0.2) (layer "F.Cu") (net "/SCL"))
 (segment (start 157 76.92) (end 157.485685 76.92) (width 0.2) (layer "F.Cu") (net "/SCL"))
 (segment (start 165 109.765685) (end 165.234315 110) (width 0.2) (layer "F.Cu") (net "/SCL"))
 (segment (start 185 97.414214) (end 162.635 75.049214) (width 0.2) (layer "F.Cu") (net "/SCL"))
 (segment (start 162.635 69.881358) (end 158.213642 65.46) (width 0.2) (layer "F.Cu") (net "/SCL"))
 (segment (start 165.234315 110) (end 184 110) (width 0.2) (layer "F.Cu") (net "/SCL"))
 (segment (start 142.225 66.685) (end 139.54 64) (width 0.2) (layer "F.Cu") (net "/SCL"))
 (segment (start 157.485685 76.92) (end 165 84.434315) (width 0.2) (layer "F.Cu") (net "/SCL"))
 (segment (start 162.635 75.049214) (end 162.635 69.881358) (width 0.2) (layer "F.Cu") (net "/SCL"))
 (segment (start 118 73.3) (end 130.24 73.3) (width 0.2) (layer "B.Cu") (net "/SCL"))
 (segment (start 130.24 73.3) (end 139.54 64) (width 0.2) (layer "B.Cu") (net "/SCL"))
 (segment (start 164 111) (end 185 111) (width 0.2) (layer "F.Cu") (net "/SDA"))
 (segment (start 165 70.176654) (end 164.261346 69.438) (width 0.2) (layer "F.Cu") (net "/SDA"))
 (segment (start 175.4 87.248528) (end 175.4 86.751472) (width 0.2) (layer "F.Cu") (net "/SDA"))
 (segment (start 157 79.46) (end 155.625 79.46) (width 0.2) (layer "F.Cu") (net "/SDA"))
 (segment (start 162.757328 69.438) (end 159 65.680672) (width 0.2) (layer "F.Cu") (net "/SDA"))
 (segment (start 164 84) (end 164 111) (width 0.2) (layer "F.Cu") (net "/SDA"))
 (segment (start 175.4 86.751472) (end 165 76.351472) (width 0.2) (layer "F.Cu") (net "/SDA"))
 (segment (start 186 110) (end 186 89) (width 0.2) (layer "F.Cu") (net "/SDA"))
 (segment (start 143.495 62.585) (end 142.08 64) (width 0.2) (layer "F.Cu") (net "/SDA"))
 (segment (start 165 76.351472) (end 165 70.176654) (width 0.2) (layer "F.Cu") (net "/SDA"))
 (segment (start 159 62.585) (end 143.495 62.585) (width 0.2) (layer "F.Cu") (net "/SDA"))
 (segment (start 159.46 79.46) (end 164 84) (width 0.2) (layer "F.Cu") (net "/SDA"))
 (segment (start 164.261346 69.438) (end 162.757328 69.438) (width 0.2) (layer "F.Cu") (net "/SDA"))
 (segment (start 185 111) (end 186 110) (width 0.2) (layer "F.Cu") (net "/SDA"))
 (segment (start 157 79.46) (end 159.46 79.46) (width 0.2) (layer "F.Cu") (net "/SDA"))
 (segment (start 159 65.680672) (end 159 62.585) (width 0.2) (layer "F.Cu") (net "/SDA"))
 (segment (start 185 88) (end 176.151472 88) (width 0.2) (layer "F.Cu") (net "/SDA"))
 (segment (start 176.151472 88) (end 175.4 87.248528) (width 0.2) (layer "F.Cu") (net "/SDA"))
 (segment (start 186 89) (end 185 88) (width 0.2) (layer "F.Cu") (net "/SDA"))
 (segment (start 130.24 75.84) (end 142.08 64) (width 0.2) (layer "B.Cu") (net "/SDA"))
 (segment (start 118 75.84) (end 130.24 75.84) (width 0.2) (layer "B.Cu") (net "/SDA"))
 (segment (start 171.79 69.3) (end 170.778 68.288) (width 0.2) (layer "F.Cu") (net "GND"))
 (segment (start 170.778 68.288) (end 166.325 68.288) (width 0.2) (layer "F.Cu") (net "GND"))
 (segment (start 173.165 69.3) (end 164.865 61) (width 0.2) (layer "F.Cu") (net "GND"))
 (segment (start 173.165 69.3) (end 171.79 69.3) (width 0.2) (layer "F.Cu") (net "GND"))
 (segment (start 137.46 61) (end 134.46 64) (width 0.2) (layer "F.Cu") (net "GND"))
 (segment (start 164.865 61) (end 137.46 61) (width 0.2) (layer "F.Cu") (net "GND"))
 (segment (start 118 70.76) (end 124.318138 70.76) (width 0.2) (layer "B.Cu") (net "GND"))
 (segment (start 111.68 77.08) (end 118 70.76) (width 0.2) (layer "B.Cu") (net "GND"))
 (segment (start 124.318138 70.76) (end 131.078138 64) (width 0.2) (layer "B.Cu") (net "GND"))
 (segment (start 107 77.08) (end 111.68 77.08) (width 0.2) (layer "B.Cu") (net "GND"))
 (segment (start 99.11 97.46) (end 107 89.57) (width 0.2) (layer "B.Cu") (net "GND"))
 (segment (start 99.11 97.46) (end 172.11 97.46) (width 0.2) (layer "B.Cu") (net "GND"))
 (segment (start 131.078138 64) (end 134.46 64) (width 0.2) (layer "B.Cu") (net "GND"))
 (segment (start 107 89.57) (end 107 77.08) (width 0.2) (layer "B.Cu") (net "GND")))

